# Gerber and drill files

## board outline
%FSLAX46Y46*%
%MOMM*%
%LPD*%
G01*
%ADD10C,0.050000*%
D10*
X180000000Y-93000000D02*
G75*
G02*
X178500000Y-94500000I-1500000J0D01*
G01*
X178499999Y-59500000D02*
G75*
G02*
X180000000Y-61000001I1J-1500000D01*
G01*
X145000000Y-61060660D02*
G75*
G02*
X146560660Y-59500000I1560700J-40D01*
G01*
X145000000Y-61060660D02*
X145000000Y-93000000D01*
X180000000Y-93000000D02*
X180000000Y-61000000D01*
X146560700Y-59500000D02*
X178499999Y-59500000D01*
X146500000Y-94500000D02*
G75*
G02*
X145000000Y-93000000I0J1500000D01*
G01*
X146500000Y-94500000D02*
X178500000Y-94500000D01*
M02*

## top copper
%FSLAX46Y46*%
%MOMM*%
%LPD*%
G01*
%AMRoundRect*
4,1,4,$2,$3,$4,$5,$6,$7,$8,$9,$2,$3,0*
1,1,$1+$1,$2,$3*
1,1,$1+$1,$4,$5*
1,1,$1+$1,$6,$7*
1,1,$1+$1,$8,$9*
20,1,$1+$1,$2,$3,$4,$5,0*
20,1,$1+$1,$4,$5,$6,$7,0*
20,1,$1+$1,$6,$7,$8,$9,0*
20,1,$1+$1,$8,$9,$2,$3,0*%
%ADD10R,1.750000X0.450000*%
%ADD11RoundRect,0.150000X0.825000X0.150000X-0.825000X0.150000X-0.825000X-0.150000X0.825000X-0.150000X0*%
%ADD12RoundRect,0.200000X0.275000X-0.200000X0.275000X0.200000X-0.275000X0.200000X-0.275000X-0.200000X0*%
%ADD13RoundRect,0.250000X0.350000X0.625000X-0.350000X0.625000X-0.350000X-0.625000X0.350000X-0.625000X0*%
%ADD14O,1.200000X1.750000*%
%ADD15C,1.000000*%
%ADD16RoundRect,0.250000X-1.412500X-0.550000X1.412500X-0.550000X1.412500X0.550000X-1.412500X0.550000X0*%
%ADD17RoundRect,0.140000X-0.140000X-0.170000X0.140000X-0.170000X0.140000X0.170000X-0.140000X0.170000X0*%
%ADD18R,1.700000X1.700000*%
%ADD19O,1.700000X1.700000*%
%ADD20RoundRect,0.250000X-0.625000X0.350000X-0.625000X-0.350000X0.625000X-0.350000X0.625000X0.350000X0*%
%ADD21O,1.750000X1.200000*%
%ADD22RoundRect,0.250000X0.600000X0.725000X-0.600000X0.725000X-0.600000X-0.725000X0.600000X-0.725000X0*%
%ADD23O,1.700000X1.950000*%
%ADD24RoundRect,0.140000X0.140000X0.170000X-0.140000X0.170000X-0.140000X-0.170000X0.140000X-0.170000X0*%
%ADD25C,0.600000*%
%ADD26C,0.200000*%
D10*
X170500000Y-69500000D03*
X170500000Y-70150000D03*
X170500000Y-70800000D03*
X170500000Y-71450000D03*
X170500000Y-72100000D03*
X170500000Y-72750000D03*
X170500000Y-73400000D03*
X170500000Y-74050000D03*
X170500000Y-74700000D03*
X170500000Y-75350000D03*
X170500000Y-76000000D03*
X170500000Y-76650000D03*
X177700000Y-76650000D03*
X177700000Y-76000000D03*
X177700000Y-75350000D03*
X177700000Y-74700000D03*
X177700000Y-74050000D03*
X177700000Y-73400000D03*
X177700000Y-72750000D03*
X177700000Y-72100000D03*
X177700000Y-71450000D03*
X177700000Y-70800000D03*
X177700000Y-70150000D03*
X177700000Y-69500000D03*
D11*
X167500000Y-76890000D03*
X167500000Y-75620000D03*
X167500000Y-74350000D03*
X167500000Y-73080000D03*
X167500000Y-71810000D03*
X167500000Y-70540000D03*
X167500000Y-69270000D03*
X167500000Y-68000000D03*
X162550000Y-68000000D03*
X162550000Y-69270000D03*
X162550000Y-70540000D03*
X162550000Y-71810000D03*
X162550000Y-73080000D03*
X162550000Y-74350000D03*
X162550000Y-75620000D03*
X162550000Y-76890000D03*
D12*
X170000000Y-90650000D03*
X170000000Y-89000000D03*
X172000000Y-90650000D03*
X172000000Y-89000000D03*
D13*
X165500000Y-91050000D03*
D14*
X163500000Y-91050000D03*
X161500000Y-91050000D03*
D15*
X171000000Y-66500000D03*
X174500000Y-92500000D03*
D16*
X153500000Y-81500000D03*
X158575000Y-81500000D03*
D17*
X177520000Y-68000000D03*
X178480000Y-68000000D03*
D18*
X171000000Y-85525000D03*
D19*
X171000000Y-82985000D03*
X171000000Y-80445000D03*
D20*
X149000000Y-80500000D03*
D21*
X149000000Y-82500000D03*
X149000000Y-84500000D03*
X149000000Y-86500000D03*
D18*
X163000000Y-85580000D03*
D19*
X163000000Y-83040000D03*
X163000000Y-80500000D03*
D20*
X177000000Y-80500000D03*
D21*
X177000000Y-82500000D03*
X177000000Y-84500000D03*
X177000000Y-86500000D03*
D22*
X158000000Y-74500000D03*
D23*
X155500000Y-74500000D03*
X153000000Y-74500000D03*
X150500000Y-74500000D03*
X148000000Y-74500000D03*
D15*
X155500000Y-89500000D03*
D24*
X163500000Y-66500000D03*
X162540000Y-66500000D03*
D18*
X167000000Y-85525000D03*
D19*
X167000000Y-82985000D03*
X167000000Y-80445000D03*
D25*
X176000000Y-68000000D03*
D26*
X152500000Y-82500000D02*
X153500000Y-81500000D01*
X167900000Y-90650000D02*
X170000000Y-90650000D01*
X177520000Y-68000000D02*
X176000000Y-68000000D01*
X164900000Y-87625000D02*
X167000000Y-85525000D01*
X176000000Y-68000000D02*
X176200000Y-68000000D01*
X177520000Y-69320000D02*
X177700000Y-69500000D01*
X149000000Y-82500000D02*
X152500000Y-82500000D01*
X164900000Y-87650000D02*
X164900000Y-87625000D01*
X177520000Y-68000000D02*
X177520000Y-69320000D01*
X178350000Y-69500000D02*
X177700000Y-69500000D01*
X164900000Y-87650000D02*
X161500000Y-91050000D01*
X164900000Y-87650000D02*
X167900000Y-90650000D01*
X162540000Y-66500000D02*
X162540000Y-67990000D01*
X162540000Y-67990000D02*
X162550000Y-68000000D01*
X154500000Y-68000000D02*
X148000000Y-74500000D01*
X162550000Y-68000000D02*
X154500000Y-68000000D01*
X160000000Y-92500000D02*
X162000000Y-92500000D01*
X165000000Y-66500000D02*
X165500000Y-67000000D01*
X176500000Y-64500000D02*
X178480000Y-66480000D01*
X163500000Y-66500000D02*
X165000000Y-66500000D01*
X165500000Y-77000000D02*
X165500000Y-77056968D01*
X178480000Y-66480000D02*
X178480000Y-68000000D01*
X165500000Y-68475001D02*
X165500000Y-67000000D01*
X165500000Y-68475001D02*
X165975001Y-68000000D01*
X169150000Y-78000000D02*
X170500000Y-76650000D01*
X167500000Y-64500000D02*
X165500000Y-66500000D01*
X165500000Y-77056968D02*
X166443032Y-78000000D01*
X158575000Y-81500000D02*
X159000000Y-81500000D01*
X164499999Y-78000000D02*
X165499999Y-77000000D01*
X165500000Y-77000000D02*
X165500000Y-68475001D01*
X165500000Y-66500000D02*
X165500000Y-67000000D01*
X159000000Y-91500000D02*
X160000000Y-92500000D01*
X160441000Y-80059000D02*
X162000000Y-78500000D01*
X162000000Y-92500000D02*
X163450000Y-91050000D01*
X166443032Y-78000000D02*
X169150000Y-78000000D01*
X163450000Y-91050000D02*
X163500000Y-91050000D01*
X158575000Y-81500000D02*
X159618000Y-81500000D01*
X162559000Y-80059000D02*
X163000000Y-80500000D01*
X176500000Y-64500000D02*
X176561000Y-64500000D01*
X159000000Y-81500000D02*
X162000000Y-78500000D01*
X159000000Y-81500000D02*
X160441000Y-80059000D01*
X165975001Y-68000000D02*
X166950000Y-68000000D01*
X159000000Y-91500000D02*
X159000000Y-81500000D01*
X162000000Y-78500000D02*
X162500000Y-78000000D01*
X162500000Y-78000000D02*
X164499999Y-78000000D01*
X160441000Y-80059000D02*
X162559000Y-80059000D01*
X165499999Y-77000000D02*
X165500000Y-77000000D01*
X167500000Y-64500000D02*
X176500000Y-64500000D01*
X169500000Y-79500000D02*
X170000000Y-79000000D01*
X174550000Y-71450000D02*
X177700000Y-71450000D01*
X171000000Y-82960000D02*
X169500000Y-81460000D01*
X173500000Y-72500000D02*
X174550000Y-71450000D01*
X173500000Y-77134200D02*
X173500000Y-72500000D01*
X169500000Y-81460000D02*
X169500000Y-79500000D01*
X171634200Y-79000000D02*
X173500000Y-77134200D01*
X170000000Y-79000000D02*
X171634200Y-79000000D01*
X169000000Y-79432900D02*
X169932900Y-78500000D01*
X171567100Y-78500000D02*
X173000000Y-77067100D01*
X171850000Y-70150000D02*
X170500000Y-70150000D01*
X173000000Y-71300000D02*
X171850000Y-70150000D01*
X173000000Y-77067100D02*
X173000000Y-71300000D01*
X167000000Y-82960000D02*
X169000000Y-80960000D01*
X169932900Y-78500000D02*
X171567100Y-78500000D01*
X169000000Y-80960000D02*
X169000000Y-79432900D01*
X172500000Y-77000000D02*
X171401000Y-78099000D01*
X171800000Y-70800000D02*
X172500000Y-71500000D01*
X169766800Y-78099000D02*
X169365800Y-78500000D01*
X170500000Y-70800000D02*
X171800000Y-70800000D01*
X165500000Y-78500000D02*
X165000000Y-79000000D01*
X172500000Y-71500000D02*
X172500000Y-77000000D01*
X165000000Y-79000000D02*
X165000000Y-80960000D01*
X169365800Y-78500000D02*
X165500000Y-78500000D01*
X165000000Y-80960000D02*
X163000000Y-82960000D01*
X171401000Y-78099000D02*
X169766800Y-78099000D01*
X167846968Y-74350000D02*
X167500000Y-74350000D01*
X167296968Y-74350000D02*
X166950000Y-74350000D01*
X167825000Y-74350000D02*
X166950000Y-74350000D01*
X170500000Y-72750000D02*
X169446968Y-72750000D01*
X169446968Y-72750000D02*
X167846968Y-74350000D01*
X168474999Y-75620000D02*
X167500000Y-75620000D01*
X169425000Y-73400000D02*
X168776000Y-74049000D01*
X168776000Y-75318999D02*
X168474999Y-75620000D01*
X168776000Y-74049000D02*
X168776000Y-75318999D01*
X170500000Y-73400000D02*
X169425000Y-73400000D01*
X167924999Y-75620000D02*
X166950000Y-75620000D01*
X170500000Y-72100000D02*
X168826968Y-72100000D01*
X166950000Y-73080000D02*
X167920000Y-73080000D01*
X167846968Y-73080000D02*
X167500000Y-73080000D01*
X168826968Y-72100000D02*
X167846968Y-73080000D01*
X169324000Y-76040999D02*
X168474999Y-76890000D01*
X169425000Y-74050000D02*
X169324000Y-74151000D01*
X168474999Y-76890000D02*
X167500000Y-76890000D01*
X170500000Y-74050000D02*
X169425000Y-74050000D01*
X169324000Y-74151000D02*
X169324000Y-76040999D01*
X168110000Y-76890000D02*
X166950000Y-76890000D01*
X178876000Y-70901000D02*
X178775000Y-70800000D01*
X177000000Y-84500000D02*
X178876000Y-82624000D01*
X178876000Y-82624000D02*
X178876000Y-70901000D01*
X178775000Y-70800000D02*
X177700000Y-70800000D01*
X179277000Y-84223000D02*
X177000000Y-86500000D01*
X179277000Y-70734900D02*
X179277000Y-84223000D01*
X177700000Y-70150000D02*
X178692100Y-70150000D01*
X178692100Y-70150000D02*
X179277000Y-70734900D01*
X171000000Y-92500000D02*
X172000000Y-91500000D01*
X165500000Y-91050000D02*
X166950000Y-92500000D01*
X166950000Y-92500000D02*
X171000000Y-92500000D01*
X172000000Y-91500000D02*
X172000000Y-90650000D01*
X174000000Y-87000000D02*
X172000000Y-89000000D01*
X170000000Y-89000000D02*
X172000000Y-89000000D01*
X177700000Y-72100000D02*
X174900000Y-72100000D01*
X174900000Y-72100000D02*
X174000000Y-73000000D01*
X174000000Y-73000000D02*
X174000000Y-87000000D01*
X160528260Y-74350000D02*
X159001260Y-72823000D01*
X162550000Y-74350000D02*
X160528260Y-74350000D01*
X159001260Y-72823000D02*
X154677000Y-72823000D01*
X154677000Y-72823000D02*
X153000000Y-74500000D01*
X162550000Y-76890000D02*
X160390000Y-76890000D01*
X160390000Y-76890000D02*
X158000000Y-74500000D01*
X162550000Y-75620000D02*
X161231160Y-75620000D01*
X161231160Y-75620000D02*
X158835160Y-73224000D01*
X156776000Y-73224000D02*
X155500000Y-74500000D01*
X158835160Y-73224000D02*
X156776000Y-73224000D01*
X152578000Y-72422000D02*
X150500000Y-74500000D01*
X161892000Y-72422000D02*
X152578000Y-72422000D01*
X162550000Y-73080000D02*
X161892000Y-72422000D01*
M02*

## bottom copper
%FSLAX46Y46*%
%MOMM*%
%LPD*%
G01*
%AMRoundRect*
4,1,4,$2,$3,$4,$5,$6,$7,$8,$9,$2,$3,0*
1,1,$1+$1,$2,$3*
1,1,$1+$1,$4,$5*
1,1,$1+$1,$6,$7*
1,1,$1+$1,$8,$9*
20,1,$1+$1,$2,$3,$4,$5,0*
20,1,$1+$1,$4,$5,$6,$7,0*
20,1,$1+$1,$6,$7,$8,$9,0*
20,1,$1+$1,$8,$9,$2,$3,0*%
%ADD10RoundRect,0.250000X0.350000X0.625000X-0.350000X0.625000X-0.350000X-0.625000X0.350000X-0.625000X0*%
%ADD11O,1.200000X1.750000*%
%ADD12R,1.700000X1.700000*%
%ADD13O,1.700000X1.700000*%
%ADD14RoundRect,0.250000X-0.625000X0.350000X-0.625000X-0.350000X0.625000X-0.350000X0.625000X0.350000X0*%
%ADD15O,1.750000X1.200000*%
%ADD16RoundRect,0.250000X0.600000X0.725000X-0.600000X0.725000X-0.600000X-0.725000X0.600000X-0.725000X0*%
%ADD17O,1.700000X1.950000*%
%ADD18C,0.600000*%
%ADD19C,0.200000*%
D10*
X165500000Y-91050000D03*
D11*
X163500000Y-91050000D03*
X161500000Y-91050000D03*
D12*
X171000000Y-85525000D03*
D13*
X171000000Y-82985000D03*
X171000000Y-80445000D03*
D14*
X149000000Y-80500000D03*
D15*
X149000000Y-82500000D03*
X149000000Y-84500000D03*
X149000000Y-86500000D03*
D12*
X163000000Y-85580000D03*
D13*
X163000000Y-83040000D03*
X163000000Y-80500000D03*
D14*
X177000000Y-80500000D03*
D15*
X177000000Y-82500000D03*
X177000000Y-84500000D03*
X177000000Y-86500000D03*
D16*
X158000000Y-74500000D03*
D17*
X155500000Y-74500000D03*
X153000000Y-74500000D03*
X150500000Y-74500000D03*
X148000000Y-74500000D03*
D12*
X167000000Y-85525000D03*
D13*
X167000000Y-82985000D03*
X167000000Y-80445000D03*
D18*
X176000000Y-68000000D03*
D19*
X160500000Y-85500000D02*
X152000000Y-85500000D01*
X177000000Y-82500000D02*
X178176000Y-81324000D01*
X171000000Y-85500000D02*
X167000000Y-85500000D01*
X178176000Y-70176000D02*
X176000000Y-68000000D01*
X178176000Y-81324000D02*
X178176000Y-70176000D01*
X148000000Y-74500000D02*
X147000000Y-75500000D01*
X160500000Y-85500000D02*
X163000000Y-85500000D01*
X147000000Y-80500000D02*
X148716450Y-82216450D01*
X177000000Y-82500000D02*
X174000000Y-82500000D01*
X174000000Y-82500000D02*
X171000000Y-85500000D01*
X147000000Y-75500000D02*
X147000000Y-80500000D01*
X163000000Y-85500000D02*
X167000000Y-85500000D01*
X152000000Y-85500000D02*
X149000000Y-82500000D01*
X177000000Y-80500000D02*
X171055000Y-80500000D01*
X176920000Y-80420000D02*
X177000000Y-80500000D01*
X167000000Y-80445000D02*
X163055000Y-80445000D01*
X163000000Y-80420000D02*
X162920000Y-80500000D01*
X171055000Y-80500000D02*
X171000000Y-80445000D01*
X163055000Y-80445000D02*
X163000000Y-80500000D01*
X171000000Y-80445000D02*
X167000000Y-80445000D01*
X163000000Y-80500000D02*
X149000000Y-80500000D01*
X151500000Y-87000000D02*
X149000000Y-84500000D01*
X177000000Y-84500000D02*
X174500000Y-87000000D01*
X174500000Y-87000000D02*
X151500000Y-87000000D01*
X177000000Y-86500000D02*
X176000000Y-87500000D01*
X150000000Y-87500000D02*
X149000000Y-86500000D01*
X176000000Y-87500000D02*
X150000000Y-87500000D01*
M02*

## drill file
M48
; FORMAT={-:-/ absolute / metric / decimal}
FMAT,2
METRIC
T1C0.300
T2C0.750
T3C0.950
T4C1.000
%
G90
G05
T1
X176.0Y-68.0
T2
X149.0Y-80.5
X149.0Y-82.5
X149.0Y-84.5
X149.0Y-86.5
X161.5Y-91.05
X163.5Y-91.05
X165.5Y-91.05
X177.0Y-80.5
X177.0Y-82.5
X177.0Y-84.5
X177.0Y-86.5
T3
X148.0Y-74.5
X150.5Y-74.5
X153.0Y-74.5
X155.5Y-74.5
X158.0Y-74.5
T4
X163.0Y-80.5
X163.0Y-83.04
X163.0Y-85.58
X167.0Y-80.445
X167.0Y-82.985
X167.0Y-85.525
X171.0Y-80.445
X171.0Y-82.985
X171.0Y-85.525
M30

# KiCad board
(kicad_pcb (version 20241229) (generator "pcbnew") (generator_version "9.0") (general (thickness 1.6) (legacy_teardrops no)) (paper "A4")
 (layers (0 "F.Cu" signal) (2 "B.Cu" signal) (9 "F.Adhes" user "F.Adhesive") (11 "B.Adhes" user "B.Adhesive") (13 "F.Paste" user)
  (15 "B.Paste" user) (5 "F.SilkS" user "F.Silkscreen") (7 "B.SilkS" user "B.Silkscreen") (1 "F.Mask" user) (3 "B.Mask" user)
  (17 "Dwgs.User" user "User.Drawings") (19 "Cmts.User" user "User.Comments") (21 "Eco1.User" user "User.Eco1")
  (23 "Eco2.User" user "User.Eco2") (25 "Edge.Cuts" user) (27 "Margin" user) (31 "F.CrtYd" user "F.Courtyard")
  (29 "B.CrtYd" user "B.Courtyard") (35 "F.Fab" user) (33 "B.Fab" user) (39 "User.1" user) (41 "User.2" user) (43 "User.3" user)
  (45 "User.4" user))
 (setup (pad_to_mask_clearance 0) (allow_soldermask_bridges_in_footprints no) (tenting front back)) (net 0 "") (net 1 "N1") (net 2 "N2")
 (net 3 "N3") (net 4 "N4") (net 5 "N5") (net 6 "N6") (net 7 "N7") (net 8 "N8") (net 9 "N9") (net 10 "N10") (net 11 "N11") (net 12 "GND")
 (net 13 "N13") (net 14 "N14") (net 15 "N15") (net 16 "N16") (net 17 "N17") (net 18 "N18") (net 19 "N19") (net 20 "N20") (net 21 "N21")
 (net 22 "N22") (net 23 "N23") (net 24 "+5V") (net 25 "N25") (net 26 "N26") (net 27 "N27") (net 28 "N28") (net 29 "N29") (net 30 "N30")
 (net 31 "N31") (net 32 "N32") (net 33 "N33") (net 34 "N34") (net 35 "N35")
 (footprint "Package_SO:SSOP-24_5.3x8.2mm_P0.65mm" (layer "F.Cu") (at 174.1 73.075)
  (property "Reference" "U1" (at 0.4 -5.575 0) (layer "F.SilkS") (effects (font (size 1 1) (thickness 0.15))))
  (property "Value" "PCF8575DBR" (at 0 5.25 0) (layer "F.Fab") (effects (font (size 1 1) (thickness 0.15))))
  (pad "1" smd rect (at -3.6 -3.575) (size 1.75 0.45) (layers "F.Cu" "F.Mask" "F.Paste") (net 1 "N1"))
  (pad "2" smd rect (at -3.6 -2.925) (size 1.75 0.45) (layers "F.Cu" "F.Mask" "F.Paste") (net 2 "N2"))
  (pad "3" smd rect (at -3.6 -2.275) (size 1.75 0.45) (layers "F.Cu" "F.Mask" "F.Paste") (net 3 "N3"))
  (pad "4" smd rect (at -3.6 -1.625) (size 1.75 0.45) (layers "F.Cu" "F.Mask" "F.Paste") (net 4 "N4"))
  (pad "5" smd rect (at -3.6 -0.975) (size 1.75 0.45) (layers "F.Cu" "F.Mask" "F.Paste") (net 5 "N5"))
  (pad "6" smd rect (at -3.6 -0.325) (size 1.75 0.45) (layers "F.Cu" "F.Mask" "F.Paste") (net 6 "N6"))
  (pad "7" smd rect (at -3.6 0.325) (size 1.75 0.45) (layers "F.Cu" "F.Mask" "F.Paste") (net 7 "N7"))
  (pad "8" smd rect (at -3.6 0.975) (size 1.75 0.45) (layers "F.Cu" "F.Mask" "F.Paste") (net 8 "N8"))
  (pad "9" smd rect (at -3.6 1.625) (size 1.75 0.45) (layers "F.Cu" "F.Mask" "F.Paste") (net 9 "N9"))
  (pad "10" smd rect (at -3.6 2.275) (size 1.75 0.45) (layers "F.Cu" "F.Mask" "F.Paste") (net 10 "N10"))
  (pad "11" smd rect (at -3.6 2.925) (size 1.75 0.45) (layers "F.Cu" "F.Mask" "F.Paste") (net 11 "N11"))
  (pad "12" smd rect (at -3.6 3.575) (size 1.75 0.45) (layers "F.Cu" "F.Mask" "F.Paste") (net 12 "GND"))
  (pad "13" smd rect (at 3.6 3.575) (size 1.75 0.45) (layers "F.Cu" "F.Mask" "F.Paste") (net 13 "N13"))
  (pad "14" smd rect (at 3.6 2.925) (size 1.75 0.45) (layers "F.Cu" "F.Mask" "F.Paste") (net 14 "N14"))
  (pad "15" smd rect (at 3.6 2.275) (size 1.75 0.45) (layers "F.Cu" "F.Mask" "F.Paste") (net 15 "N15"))
  (pad "16" smd rect (at 3.6 1.625) (size 1.75 0.45) (layers "F.Cu" "F.Mask" "F.Paste") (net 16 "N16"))
  (pad "17" smd rect (at 3.6 0.975) (size 1.75 0.45) (layers "F.Cu" "F.Mask" "F.Paste") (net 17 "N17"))
  (pad "18" smd rect (at 3.6 0.325) (size 1.75 0.45) (layers "F.Cu" "F.Mask" "F.Paste") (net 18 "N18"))
  (pad "19" smd rect (at 3.6 -0.325) (size 1.75 0.45) (layers "F.Cu" "F.Mask" "F.Paste") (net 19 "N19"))
  (pad "20" smd rect (at 3.6 -0.975) (size 1.75 0.45) (layers "F.Cu" "F.Mask" "F.Paste") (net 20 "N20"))
  (pad "21" smd rect (at 3.6 -1.625) (size 1.75 0.45) (layers "F.Cu" "F.Mask" "F.Paste") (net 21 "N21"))
  (pad "22" smd rect (at 3.6 -2.275) (size 1.75 0.45) (layers "F.Cu" "F.Mask" "F.Paste") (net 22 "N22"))
  (pad "23" smd rect (at 3.6 -2.925) (size 1.75 0.45) (layers "F.Cu" "F.Mask" "F.Paste") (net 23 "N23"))
  (pad "24" smd rect (at 3.6 -3.575) (size 1.75 0.45) (layers "F.Cu" "F.Mask" "F.Paste") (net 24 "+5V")))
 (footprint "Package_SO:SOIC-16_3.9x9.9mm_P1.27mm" (layer "F.Cu") (at 165.025 72.445 180)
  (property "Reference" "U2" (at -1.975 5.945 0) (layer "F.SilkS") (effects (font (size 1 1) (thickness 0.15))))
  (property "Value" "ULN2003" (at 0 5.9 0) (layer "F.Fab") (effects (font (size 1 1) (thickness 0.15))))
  (pad "1" smd roundrect (at -2.475 -4.445 180) (size 1.95 0.6) (layers "F.Cu" "F.Mask" "F.Paste") (roundrect_rratio 0.25) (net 8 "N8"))
  (pad "2" smd roundrect (at -2.475 -3.175 180) (size 1.95 0.6) (layers "F.Cu" "F.Mask" "F.Paste") (roundrect_rratio 0.25) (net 7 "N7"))
  (pad "3" smd roundrect (at -2.475 -1.905 180) (size 1.95 0.6) (layers "F.Cu" "F.Mask" "F.Paste") (roundrect_rratio 0.25) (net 6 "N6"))
  (pad "4" smd roundrect (at -2.475 -0.635 180) (size 1.95 0.6) (layers "F.Cu" "F.Mask" "F.Paste") (roundrect_rratio 0.25) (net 5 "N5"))
  (pad "5" smd roundrect (at -2.475 0.635 180) (size 1.95 0.6) (layers "F.Cu" "F.Mask" "F.Paste") (roundrect_rratio 0.25) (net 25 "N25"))
  (pad "6" smd roundrect (at -2.475 1.905 180) (size 1.95 0.6) (layers "F.Cu" "F.Mask" "F.Paste") (roundrect_rratio 0.25) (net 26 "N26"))
  (pad "7" smd roundrect (at -2.475 3.175 180) (size 1.95 0.6) (layers "F.Cu" "F.Mask" "F.Paste") (roundrect_rratio 0.25) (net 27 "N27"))
  (pad "8" smd roundrect (at -2.475 4.445 180) (size 1.95 0.6) (layers "F.Cu" "F.Mask" "F.Paste") (roundrect_rratio 0.25) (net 12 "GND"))
  (pad "9" smd roundrect (at 2.475 4.445 180) (size 1.95 0.6) (layers "F.Cu" "F.Mask" "F.Paste") (roundrect_rratio 0.25) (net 24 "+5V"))
  (pad "10" smd roundrect (at 2.475 3.175 180) (size 1.95 0.6) (layers "F.Cu" "F.Mask" "F.Paste") (roundrect_rratio 0.25) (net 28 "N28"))
  (pad "11" smd roundrect (at 2.475 1.905 180) (size 1.95 0.6) (layers "F.Cu" "F.Mask" "F.Paste") (roundrect_rratio 0.25) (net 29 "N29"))
  (pad "12" smd roundrect (at 2.475 0.635 180) (size 1.95 0.6) (layers "F.Cu" "F.Mask" "F.Paste") (roundrect_rratio 0.25) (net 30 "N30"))
  (pad "13" smd roundrect (at 2.475 -0.635 180) (size 1.95 0.6) (layers "F.Cu" "F.Mask" "F.Paste") (roundrect_rratio 0.25) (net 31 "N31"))
  (pad "14" smd roundrect (at 2.475 -1.905 180) (size 1.95 0.6) (layers "F.Cu" "F.Mask" "F.Paste") (roundrect_rratio 0.25) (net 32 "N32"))
  (pad "15" smd roundrect (at 2.475 -3.175 180) (size 1.95 0.6) (layers "F.Cu" "F.Mask" "F.Paste") (roundrect_rratio 0.25) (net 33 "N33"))
  (pad "16" smd roundrect (at 2.475 -4.445 180) (size 1.95 0.6) (layers "F.Cu" "F.Mask" "F.Paste") (roundrect_rratio 0.25) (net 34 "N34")))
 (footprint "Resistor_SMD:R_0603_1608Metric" (layer "F.Cu") (at 170 89.825 90)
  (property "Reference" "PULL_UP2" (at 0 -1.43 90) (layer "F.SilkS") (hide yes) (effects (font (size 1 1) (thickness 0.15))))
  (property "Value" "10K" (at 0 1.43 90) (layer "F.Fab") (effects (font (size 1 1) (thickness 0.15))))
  (pad "1" smd roundrect (at -0.825 0 90) (size 0.8 0.95) (layers "F.Cu" "F.Mask" "F.Paste") (roundrect_rratio 0.25) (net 24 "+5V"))
  (pad "2" smd roundrect (at 0.825 0 90) (size 0.8 0.95) (layers "F.Cu" "F.Mask" "F.Paste") (roundrect_rratio 0.25) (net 20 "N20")))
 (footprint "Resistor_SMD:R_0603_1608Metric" (layer "F.Cu") (at 172 89.825 90)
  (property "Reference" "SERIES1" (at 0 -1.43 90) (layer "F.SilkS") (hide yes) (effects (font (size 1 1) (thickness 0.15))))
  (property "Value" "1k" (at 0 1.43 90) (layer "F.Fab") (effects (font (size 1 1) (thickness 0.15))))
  (pad "1" smd roundrect (at -0.825 0 90) (size 0.8 0.95) (layers "F.Cu" "F.Mask" "F.Paste") (roundrect_rratio 0.25) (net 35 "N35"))
  (pad "2" smd roundrect (at 0.825 0 90) (size 0.8 0.95) (layers "F.Cu" "F.Mask" "F.Paste") (roundrect_rratio 0.25) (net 20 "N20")))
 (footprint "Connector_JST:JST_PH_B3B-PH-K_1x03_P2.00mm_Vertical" (layer "F.Cu") (at 165.5 91.05 180)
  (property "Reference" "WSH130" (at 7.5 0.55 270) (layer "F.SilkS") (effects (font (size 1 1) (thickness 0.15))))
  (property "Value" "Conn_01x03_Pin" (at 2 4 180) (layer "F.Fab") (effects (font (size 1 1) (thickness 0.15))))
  (pad "1" thru_hole roundrect (at 0 0 180) (size 1.2 1.75) (drill 0.75) (layers "*.Cu" "*.Mask") (remove_unused_layers no)
   (roundrect_rratio 0.208333) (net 35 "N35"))
  (pad "2" thru_hole oval (at 2 0 180) (size 1.2 1.75) (drill 0.75) (layers "*.Cu" "*.Mask") (remove_unused_layers no) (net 12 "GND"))
  (pad "3" thru_hole oval (at 4 0 180) (size 1.2 1.75) (drill 0.75) (layers "*.Cu" "*.Mask") (remove_unused_layers no) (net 24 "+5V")))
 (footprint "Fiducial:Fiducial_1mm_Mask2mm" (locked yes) (layer "F.Cu") (at 171 66.5)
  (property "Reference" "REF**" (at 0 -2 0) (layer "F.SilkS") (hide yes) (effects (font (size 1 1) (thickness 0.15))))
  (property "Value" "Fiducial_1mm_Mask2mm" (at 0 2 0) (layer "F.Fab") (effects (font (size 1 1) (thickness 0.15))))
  (pad "" smd circle (at 0 0) (size 1 1) (layers "F.Cu" "F.Mask") (solder_mask_margin 0.5) (clearance 0.5)))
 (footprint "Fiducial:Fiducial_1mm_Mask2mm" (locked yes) (layer "F.Cu") (at 174.5 92.5)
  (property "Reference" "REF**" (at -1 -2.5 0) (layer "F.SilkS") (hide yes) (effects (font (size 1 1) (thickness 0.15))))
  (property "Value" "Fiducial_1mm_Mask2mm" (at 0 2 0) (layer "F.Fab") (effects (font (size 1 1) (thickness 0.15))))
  (pad "" smd circle (at 0 0) (size 1 1) (layers "F.Cu" "F.Mask") (solder_mask_margin 0.5) (clearance 0.5)))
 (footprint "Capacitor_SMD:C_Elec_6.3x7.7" (layer "F.Cu") (at 156.0375 81.5)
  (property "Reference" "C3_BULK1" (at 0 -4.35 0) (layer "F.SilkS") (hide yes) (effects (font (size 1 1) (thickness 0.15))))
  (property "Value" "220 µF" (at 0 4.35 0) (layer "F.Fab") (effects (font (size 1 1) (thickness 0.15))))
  (pad "1" smd roundrect (at -2.5375 0) (size 3.325 1.6) (layers "F.Cu" "F.Mask" "F.Paste") (roundrect_rratio 0.15625) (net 24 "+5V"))
  (pad "2" smd roundrect (at 2.5375 0) (size 3.325 1.6) (layers "F.Cu" "F.Mask" "F.Paste") (roundrect_rratio 0.15625) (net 12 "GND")))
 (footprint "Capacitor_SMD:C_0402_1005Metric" (layer "F.Cu") (at 178 68)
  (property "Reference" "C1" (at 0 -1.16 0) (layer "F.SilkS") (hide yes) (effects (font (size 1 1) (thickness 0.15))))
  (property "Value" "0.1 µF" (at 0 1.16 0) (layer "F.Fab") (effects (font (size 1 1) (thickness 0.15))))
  (pad "1" smd roundrect (at -0.48 0) (size 0.56 0.62) (layers "F.Cu" "F.Mask" "F.Paste") (roundrect_rratio 0.25) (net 24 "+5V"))
  (pad "2" smd roundrect (at 0.48 0) (size 0.56 0.62) (layers "F.Cu" "F.Mask" "F.Paste") (roundrect_rratio 0.25) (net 12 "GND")))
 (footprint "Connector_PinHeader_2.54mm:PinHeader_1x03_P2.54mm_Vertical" (layer "F.Cu") (at 171 85.525 180)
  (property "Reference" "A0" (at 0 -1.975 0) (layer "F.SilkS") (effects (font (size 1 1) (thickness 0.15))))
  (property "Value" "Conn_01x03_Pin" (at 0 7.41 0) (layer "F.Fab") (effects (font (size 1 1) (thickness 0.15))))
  (pad "1" thru_hole rect (at 0 0 180) (size 1.7 1.7) (drill 1) (layers "*.Cu" "*.Mask") (remove_unused_layers no) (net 24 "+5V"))
  (pad "2" thru_hole oval (at 0 2.54 180) (size 1.7 1.7) (drill 1) (layers "*.Cu" "*.Mask") (remove_unused_layers no) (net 21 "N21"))
  (pad "3" thru_hole oval (at 0 5.08 180) (size 1.7 1.7) (drill 1) (layers "*.Cu" "*.Mask") (remove_unused_layers no) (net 12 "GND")))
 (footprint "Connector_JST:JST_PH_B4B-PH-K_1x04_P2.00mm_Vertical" (layer "F.Cu") (at 149 80.5 -90)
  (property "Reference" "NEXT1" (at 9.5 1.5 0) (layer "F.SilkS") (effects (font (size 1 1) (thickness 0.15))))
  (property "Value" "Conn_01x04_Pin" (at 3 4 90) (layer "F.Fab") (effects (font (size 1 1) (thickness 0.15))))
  (pad "1" thru_hole roundrect (at 0 0 270) (size 1.2 1.75) (drill 0.75) (layers "*.Cu" "*.Mask") (remove_unused_layers no)
   (roundrect_rratio 0.208333) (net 12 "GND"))
  (pad "2" thru_hole oval (at 2 0 270) (size 1.2 1.75) (drill 0.75) (layers "*.Cu" "*.Mask") (remove_unused_layers no) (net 24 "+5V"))
  (pad "3" thru_hole oval (at 4 0 270) (size 1.2 1.75) (drill 0.75) (layers "*.Cu" "*.Mask") (remove_unused_layers no) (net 22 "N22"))
  (pad "4" thru_hole oval (at 6 0 270) (size 1.2 1.75) (drill 0.75) (layers "*.Cu" "*.Mask") (remove_unused_layers no) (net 23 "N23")))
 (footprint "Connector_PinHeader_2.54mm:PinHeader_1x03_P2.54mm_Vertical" (layer "F.Cu") (at 163 85.58 180)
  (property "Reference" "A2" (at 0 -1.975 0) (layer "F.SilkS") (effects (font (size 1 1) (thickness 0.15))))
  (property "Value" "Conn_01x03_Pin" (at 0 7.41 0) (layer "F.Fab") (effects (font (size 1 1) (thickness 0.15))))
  (pad "1" thru_hole rect (at 0 0 180) (size 1.7 1.7) (drill 1) (layers "*.Cu" "*.Mask") (remove_unused_layers no) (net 24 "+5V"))
  (pad "2" thru_hole oval (at 0 2.54 180) (size 1.7 1.7) (drill 1) (layers "*.Cu" "*.Mask") (remove_unused_layers no) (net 3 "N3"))
  (pad "3" thru_hole oval (at 0 5.08 180) (size 1.7 1.7) (drill 1) (layers "*.Cu" "*.Mask") (remove_unused_layers no) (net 12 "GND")))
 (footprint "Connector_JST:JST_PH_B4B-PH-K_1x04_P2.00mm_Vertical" (layer "F.Cu") (at 177 80.5 -90)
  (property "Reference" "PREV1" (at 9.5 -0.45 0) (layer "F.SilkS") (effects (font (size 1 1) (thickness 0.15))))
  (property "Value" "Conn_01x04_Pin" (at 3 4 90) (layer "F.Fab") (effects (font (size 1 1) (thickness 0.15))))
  (pad "1" thru_hole roundrect (at 0 0 270) (size 1.2 1.75) (drill 0.75) (layers "*.Cu" "*.Mask") (remove_unused_layers no)
   (roundrect_rratio 0.208333) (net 12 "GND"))
  (pad "2" thru_hole oval (at 2 0 270) (size 1.2 1.75) (drill 0.75) (layers "*.Cu" "*.Mask") (remove_unused_layers no) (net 24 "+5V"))
  (pad "3" thru_hole oval (at 4 0 270) (size 1.2 1.75) (drill 0.75) (layers "*.Cu" "*.Mask") (remove_unused_layers no) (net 22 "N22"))
  (pad "4" thru_hole oval (at 6 0 270) (size 1.2 1.75) (drill 0.75) (layers "*.Cu" "*.Mask") (remove_unused_layers no) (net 23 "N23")))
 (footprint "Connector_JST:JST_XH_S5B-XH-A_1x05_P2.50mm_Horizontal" (layer "F.Cu") (at 158 74.5 180)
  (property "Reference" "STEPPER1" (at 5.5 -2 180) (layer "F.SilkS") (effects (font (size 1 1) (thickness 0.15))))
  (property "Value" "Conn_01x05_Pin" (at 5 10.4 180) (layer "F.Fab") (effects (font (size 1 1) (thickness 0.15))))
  (pad "1" thru_hole roundrect (at 0 0 180) (size 1.7 1.95) (drill 0.95) (layers "*.Cu" "*.Mask") (remove_unused_layers no)
   (roundrect_rratio 0.147059) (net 34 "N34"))
  (pad "2" thru_hole oval (at 2.5 0 180) (size 1.7 1.95) (drill 0.95) (layers "*.Cu" "*.Mask") (remove_unused_layers no) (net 33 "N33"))
  (pad "3" thru_hole oval (at 5 0 180) (size 1.7 1.95) (drill 0.95) (layers "*.Cu" "*.Mask") (remove_unused_layers no) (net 32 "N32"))
  (pad "4" thru_hole oval (at 7.5 0 180) (size 1.7 1.95) (drill 0.95) (layers "*.Cu" "*.Mask") (remove_unused_layers no) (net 31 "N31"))
  (pad "5" thru_hole oval (at 10 0 180) (size 1.7 1.95) (drill 0.95) (layers "*.Cu" "*.Mask") (remove_unused_layers no) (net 24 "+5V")))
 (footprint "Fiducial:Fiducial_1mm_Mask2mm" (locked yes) (layer "F.Cu") (at 155.5 89.5)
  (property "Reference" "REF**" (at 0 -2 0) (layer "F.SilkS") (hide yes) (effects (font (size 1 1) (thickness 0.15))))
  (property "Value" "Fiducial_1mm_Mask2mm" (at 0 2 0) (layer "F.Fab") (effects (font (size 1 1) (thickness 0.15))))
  (pad "" smd circle (at 0 0) (size 1 1) (layers "F.Cu" "F.Mask") (solder_mask_margin 0.5) (clearance 0.5)))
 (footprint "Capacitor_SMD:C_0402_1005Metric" (layer "F.Cu") (at 163.02 66.5 180)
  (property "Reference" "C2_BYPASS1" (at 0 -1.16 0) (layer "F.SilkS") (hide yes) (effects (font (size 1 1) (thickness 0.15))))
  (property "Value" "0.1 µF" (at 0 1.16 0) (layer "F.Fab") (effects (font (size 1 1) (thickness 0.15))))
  (pad "1" smd roundrect (at -0.48 0 180) (size 0.56 0.62) (layers "F.Cu" "F.Mask" "F.Paste") (roundrect_rratio 0.25) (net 12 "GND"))
  (pad "2" smd roundrect (at 0.48 0 180) (size 0.56 0.62) (layers "F.Cu" "F.Mask" "F.Paste") (roundrect_rratio 0.25) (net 24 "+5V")))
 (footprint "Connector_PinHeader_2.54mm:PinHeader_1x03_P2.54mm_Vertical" (layer "F.Cu") (at 167 85.525 180)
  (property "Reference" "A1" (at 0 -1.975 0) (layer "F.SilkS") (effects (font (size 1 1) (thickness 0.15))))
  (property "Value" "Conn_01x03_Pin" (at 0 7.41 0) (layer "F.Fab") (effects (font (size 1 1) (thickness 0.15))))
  (pad "1" thru_hole rect (at 0 0 180) (size 1.7 1.7) (drill 1) (layers "*.Cu" "*.Mask") (remove_unused_layers no) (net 24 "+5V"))
  (pad "2" thru_hole oval (at 0 2.54 180) (size 1.7 1.7) (drill 1) (layers "*.Cu" "*.Mask") (remove_unused_layers no) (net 2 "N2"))
  (pad "3" thru_hole oval (at 0 5.08 180) (size 1.7 1.7) (drill 1) (layers "*.Cu" "*.Mask") (remove_unused_layers no) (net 12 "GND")))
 (gr_arc (start 180 93) (mid 179.56066 94.06066) (end 178.5 94.5) (stroke (width 0.05) (type default)) (layer "Edge.Cuts"))
 (gr_arc (start 178.499999 59.5) (mid 179.56066 59.93934) (end 180 61.000001) (stroke (width 0.05) (type default)) (layer "Edge.Cuts"))
 (gr_arc (start 145 61.06066) (mid 145.457107 59.957107) (end 146.56066 59.5) (stroke (width 0.05) (type default)) (layer "Edge.Cuts"))
 (gr_line (start 145 61.06066) (end 145 93) (stroke (width 0.05) (type default)) (layer "Edge.Cuts"))
 (gr_line (start 180 93) (end 180 61) (stroke (width 0.05) (type default)) (layer "Edge.Cuts"))
 (gr_line (start 146.5607 59.5) (end 178.499999 59.5) (stroke (width 0.05) (type default)) (layer "Edge.Cuts"))
 (gr_arc (start 146.5 94.5) (mid 145.43934 94.06066) (end 145 93) (stroke (width 0.05) (type default)) (layer "Edge.Cuts"))
 (gr_line (start 146.5 94.5) (end 178.5 94.5) (stroke (width 0.05) (type default)) (layer "Edge.Cuts"))
 (segment (start 152.5 82.5) (end 153.5 81.5) (width 0.2) (layer "F.Cu") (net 24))
 (segment (start 167.9 90.65) (end 170 90.65) (width 0.2) (layer "F.Cu") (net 24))
 (segment (start 177.52 68) (end 176 68) (width 0.2) (layer "F.Cu") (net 24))
 (segment (start 164.9 87.625) (end 167 85.525) (width 0.2) (layer "F.Cu") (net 24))
 (segment (start 176 68) (end 176.2 68) (width 0.2) (layer "F.Cu") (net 24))
 (segment (start 177.52 69.32) (end 177.7 69.5) (width 0.2) (layer "F.Cu") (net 24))
 (segment (start 149 82.5) (end 152.5 82.5) (width 0.2) (layer "F.Cu") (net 24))
 (segment (start 164.9 87.65) (end 164.9 87.625) (width 0.2) (layer "F.Cu") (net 24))
 (segment (start 177.52 68) (end 177.52 69.32) (width 0.2) (layer "F.Cu") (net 24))
 (segment (start 178.35 69.5) (end 177.7 69.5) (width 0.2) (layer "F.Cu") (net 24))
 (segment (start 164.9 87.65) (end 161.5 91.05) (width 0.2) (layer "F.Cu") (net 24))
 (segment (start 164.9 87.65) (end 167.9 90.65) (width 0.2) (layer "F.Cu") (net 24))
 (segment (start 162.54 66.5) (end 162.54 67.99) (width 0.2) (layer "F.Cu") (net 24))
 (segment (start 162.54 67.99) (end 162.55 68) (width 0.2) (layer "F.Cu") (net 24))
 (segment (start 154.5 68) (end 148 74.5) (width 0.2) (layer "F.Cu") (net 24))
 (segment (start 162.55 68) (end 154.5 68) (width 0.2) (layer "F.Cu") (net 24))
 (via (at 176 68) (size 0.6) (drill 0.3) (layers "F.Cu" "B.Cu") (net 24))
 (segment (start 160.5 85.5) (end 152 85.5) (width 0.2) (layer "B.Cu") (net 24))
 (segment (start 177 82.5) (end 178.176 81.324) (width 0.2) (layer "B.Cu") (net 24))
 (segment (start 171 85.5) (end 167 85.5) (width 0.2) (layer "B.Cu") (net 24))
 (segment (start 178.176 70.176) (end 176 68) (width 0.2) (layer "B.Cu") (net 24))
 (segment (start 178.176 81.324) (end 178.176 70.176) (width 0.2) (layer "B.Cu") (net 24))
 (segment (start 148 74.5) (end 147 75.5) (width 0.2) (layer "B.Cu") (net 24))
 (segment (start 160.5 85.5) (end 163 85.5) (width 0.2) (layer "B.Cu") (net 24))
 (segment (start 147 80.5) (end 148.71645 82.21645) (width 0.2) (layer "B.Cu") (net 24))
 (segment (start 177 82.5) (end 174 82.5) (width 0.2) (layer "B.Cu") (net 24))
 (segment (start 174 82.5) (end 171 85.5) (width 0.2) (layer "B.Cu") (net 24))
 (segment (start 147 75.5) (end 147 80.5) (width 0.2) (layer "B.Cu") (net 24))
 (segment (start 163 85.5) (end 167 85.5) (width 0.2) (layer "B.Cu") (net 24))
 (segment (start 152 85.5) (end 149 82.5) (width 0.2) (layer "B.Cu") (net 24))
 (segment (start 160 92.5) (end 162 92.5) (width 0.2) (layer "F.Cu") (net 12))
 (segment (start 165 66.5) (end 165.5 67) (width 0.2) (layer "F.Cu") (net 12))
 (segment (start 176.5 64.5) (end 178.48 66.48) (width 0.2) (layer "F.Cu") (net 12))
 (segment (start 163.5 66.5) (end 165 66.5) (width 0.2) (layer "F.Cu") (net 12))
 (segment (start 165.5 77) (end 165.5 77.056968) (width 0.2) (layer "F.Cu") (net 12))
 (segment (start 178.48 66.48) (end 178.48 68) (width 0.2) (layer "F.Cu") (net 12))
 (segment (start 165.5 68.475001) (end 165.5 67) (width 0.2) (layer "F.Cu") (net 12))
 (segment (start 165.5 68.475001) (end 165.975001 68) (width 0.2) (layer "F.Cu") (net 12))
 (segment (start 169.15 78) (end 170.5 76.65) (width 0.2) (layer "F.Cu") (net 12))
 (segment (start 167.5 64.5) (end 165.5 66.5) (width 0.2) (layer "F.Cu") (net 12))
 (segment (start 165.5 77.056968) (end 166.443032 78) (width 0.2) (layer "F.Cu") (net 12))
 (segment (start 158.575 81.5) (end 159 81.5) (width 0.2) (layer "F.Cu") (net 12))
 (segment (start 164.499999 78) (end 165.499999 77) (width 0.2) (layer "F.Cu") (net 12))
 (segment (start 165.5 77) (end 165.5 68.475001) (width 0.2) (layer "F.Cu") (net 12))
 (segment (start 165.5 66.5) (end 165.5 67) (width 0.2) (layer "F.Cu") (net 12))
 (segment (start 159 91.5) (end 160 92.5) (width 0.2) (layer "F.Cu") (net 12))
 (segment (start 160.441 80.059) (end 162 78.5) (width 0.2) (layer "F.Cu") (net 12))
 (segment (start 162 92.5) (end 163.45 91.05) (width 0.2) (layer "F.Cu") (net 12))
 (segment (start 166.443032 78) (end 169.15 78) (width 0.2) (layer "F.Cu") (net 12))
 (segment (start 163.45 91.05) (end 163.5 91.05) (width 0.2) (layer "F.Cu") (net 12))
 (segment (start 158.575 81.5) (end 159.618 81.5) (width 0.2) (layer "F.Cu") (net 12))
 (segment (start 162.559 80.059) (end 163 80.5) (width 0.2) (layer "F.Cu") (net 12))
 (segment (start 176.5 64.5) (end 176.561 64.5) (width 0.2) (layer "F.Cu") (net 12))
 (segment (start 159 81.5) (end 162 78.5) (width 0.2) (layer "F.Cu") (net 12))
 (segment (start 159 81.5) (end 160.441 80.059) (width 0.2) (layer "F.Cu") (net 12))
 (segment (start 165.975001 68) (end 166.95 68) (width 0.2) (layer "F.Cu") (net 12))
 (segment (start 159 91.5) (end 159 81.5) (width 0.2) (layer "F.Cu") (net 12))
 (segment (start 162 78.5) (end 162.5 78) (width 0.2) (layer "F.Cu") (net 12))
 (segment (start 162.5 78) (end 164.499999 78) (width 0.2) (layer "F.Cu") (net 12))
 (segment (start 160.441 80.059) (end 162.559 80.059) (width 0.2) (layer "F.Cu") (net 12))
 (segment (start 165.499999 77) (end 165.5 77) (width 0.2) (layer "F.Cu") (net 12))
 (segment (start 167.5 64.5) (end 176.5 64.5) (width 0.2) (layer "F.Cu") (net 12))
 (segment (start 177 80.5) (end 171.055 80.5) (width 0.2) (layer "B.Cu") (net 12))
 (segment (start 176.92 80.42) (end 177 80.5) (width 0.2) (layer "B.Cu") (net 12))
 (segment (start 167 80.445) (end 163.055 80.445) (width 0.2) (layer "B.Cu") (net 12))
 (segment (start 163 80.42) (end 162.92 80.5) (width 0.2) (layer "B.Cu") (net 12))
 (segment (start 171.055 80.5) (end 171 80.445) (width 0.2) (layer "B.Cu") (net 12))
 (segment (start 163.055 80.445) (end 163 80.5) (width 0.2) (layer "B.Cu") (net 12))
 (segment (start 171 80.445) (end 167 80.445) (width 0.2) (layer "B.Cu") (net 12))
 (segment (start 163 80.5) (end 149 80.5) (width 0.2) (layer "B.Cu") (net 12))
 (segment (start 169.5 79.5) (end 170 79) (width 0.2) (layer "F.Cu") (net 21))
 (segment (start 174.55 71.45) (end 177.7 71.45) (width 0.2) (layer "F.Cu") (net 21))
 (segment (start 171 82.96) (end 169.5 81.46) (width 0.2) (layer "F.Cu") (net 21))
 (segment (start 173.5 72.5) (end 174.55 71.45) (width 0.2) (layer "F.Cu") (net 21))
 (segment (start 173.5 77.1342) (end 173.5 72.5) (width 0.2) (layer "F.Cu") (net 21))
 (segment (start 169.5 81.46) (end 169.5 79.5) (width 0.2) (layer "F.Cu") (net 21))
 (segment (start 171.6342 79) (end 173.5 77.1342) (width 0.2) (layer "F.Cu") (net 21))
 (segment (start 170 79) (end 171.6342 79) (width 0.2) (layer "F.Cu") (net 21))
 (segment (start 169 79.4329) (end 169.9329 78.5) (width 0.2) (layer "F.Cu") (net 2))
 (segment (start 171.5671 78.5) (end 173 77.0671) (width 0.2) (layer "F.Cu") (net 2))
 (segment (start 171.85 70.15) (end 170.5 70.15) (width 0.2) (layer "F.Cu") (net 2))
 (segment (start 173 71.3) (end 171.85 70.15) (width 0.2) (layer "F.Cu") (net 2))
 (segment (start 173 77.0671) (end 173 71.3) (width 0.2) (layer "F.Cu") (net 2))
 (segment (start 167 82.96) (end 169 80.96) (width 0.2) (layer "F.Cu") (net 2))
 (segment (start 169.9329 78.5) (end 171.5671 78.5) (width 0.2) (layer "F.Cu") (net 2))
 (segment (start 169 80.96) (end 169 79.4329) (width 0.2) (layer "F.Cu") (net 2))
 (segment (start 172.5 77) (end 171.401 78.099) (width 0.2) (layer "F.Cu") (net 3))
 (segment (start 171.8 70.8) (end 172.5 71.5) (width 0.2) (layer "F.Cu") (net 3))
 (segment (start 169.7668 78.099) (end 169.3658 78.5) (width 0.2) (layer "F.Cu") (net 3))
 (segment (start 170.5 70.8) (end 171.8 70.8) (width 0.2) (layer "F.Cu") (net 3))
 (segment (start 165.5 78.5) (end 165 79) (width 0.2) (layer "F.Cu") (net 3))
 (segment (start 172.5 71.5) (end 172.5 77) (width 0.2) (layer "F.Cu") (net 3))
 (segment (start 165 79) (end 165 80.96) (width 0.2) (layer "F.Cu") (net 3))
 (segment (start 169.3658 78.5) (end 165.5 78.5) (width 0.2) (layer "F.Cu") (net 3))
 (segment (start 165 80.96) (end 163 82.96) (width 0.2) (layer "F.Cu") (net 3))
 (segment (start 171.401 78.099) (end 169.7668 78.099) (width 0.2) (layer "F.Cu") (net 3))
 (segment (start 167.846968 74.35) (end 167.5 74.35) (width 0.2) (layer "F.Cu") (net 6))
 (segment (start 167.296968 74.35) (end 166.95 74.35) (width 0.2) (layer "F.Cu") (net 6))
 (segment (start 167.825 74.35) (end 166.95 74.35) (width 0.2) (layer "F.Cu") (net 6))
 (segment (start 170.5 72.75) (end 169.446968 72.75) (width 0.2) (layer "F.Cu") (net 6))
 (segment (start 169.446968 72.75) (end 167.846968 74.35) (width 0.2) (layer "F.Cu") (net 6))
 (segment (start 168.474999 75.62) (end 167.5 75.62) (width 0.2) (layer "F.Cu") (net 7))
 (segment (start 169.425 73.4) (end 168.776 74.049) (width 0.2) (layer "F.Cu") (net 7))
 (segment (start 168.776 75.318999) (end 168.474999 75.62) (width 0.2) (layer "F.Cu") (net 7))
 (segment (start 168.776 74.049) (end 168.776 75.318999) (width 0.2) (layer "F.Cu") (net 7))
 (segment (start 170.5 73.4) (end 169.425 73.4) (width 0.2) (layer "F.Cu") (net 7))
 (segment (start 167.924999 75.62) (end 166.95 75.62) (width 0.2) (layer "F.Cu") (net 7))
 (segment (start 170.5 72.1) (end 168.826968 72.1) (width 0.2) (layer "F.Cu") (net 5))
 (segment (start 166.95 73.08) (end 167.92 73.08) (width 0.2) (layer "F.Cu") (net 5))
 (segment (start 167.846968 73.08) (end 167.5 73.08) (width 0.2) (layer "F.Cu") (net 5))
 (segment (start 168.826968 72.1) (end 167.846968 73.08) (width 0.2) (layer "F.Cu") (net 5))
 (segment (start 169.324 76.040999) (end 168.474999 76.89) (width 0.2) (layer "F.Cu") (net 8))
 (segment (start 169.425 74.05) (end 169.324 74.151) (width 0.2) (layer "F.Cu") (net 8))
 (segment (start 168.474999 76.89) (end 167.5 76.89) (width 0.2) (layer "F.Cu") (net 8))
 (segment (start 170.5 74.05) (end 169.425 74.05) (width 0.2) (layer "F.Cu") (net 8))
 (segment (start 169.324 74.151) (end 169.324 76.040999) (width 0.2) (layer "F.Cu") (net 8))
 (segment (start 168.11 76.89) (end 166.95 76.89) (width 0.2) (layer "F.Cu") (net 8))
 (segment (start 178.876 70.901) (end 178.775 70.8) (width 0.2) (layer "F.Cu") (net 22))
 (segment (start 177 84.5) (end 178.876 82.624) (width 0.2) (layer "F.Cu") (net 22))
 (segment (start 178.876 82.624) (end 178.876 70.901) (width 0.2) (layer "F.Cu") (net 22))
 (segment (start 178.775 70.8) (end 177.7 70.8) (width 0.2) (layer "F.Cu") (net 22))
 (segment (start 151.5 87) (end 149 84.5) (width 0.2) (layer "B.Cu") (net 22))
 (segment (start 177 84.5) (end 174.5 87) (width 0.2) (layer "B.Cu") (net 22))
 (segment (start 174.5 87) (end 151.5 87) (width 0.2) (layer "B.Cu") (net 22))
 (segment (start 179.277 84.223) (end 177 86.5) (width 0.2) (layer "F.Cu") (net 23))
 (segment (start 179.277 70.7349) (end 179.277 84.223) (width 0.2) (layer "F.Cu") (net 23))
 (segment (start 177.7 70.15) (end 178.6921 70.15) (width 0.2) (layer "F.Cu") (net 23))
 (segment (start 178.6921 70.15) (end 179.277 70.7349) (width 0.2) (layer "F.Cu") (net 23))
 (segment (start 177 86.5) (end 176 87.5) (width 0.2) (layer "B.Cu") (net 23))
 (segment (start 150 87.5) (end 149 86.5) (width 0.2) (layer "B.Cu") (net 23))
 (segment (start 176 87.5) (end 150 87.5) (width 0.2) (layer "B.Cu") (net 23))
 (segment (start 171 92.5) (end 172 91.5) (width 0.2) (layer "F.Cu") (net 35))
 (segment (start 165.5 91.05) (end 166.95 92.5) (width 0.2) (layer "F.Cu") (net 35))
 (segment (start 166.95 92.5) (end 171 92.5) (width 0.2) (layer "F.Cu") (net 35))
 (segment (start 172 91.5) (end 172 90.65) (width 0.2) (layer "F.Cu") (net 35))
 (segment (start 174 87) (end 172 89) (width 0.2) (layer "F.Cu") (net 20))
 (segment (start 170 89) (end 172 89) (width 0.2) (layer "F.Cu") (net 20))
 (segment (start 177.7 72.1) (end 174.9 72.1) (width 0.2) (layer "F.Cu") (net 20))
 (segment (start 174.9 72.1) (end 174 73) (width 0.2) (layer "F.Cu") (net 20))
 (segment (start 174 73) (end 174 87) (width 0.2) (layer "F.Cu") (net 20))
 (segment (start 160.52826 74.35) (end 159.00126 72.823) (width 0.2) (layer "F.Cu") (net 32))
 (segment (start 162.55 74.35) (end 160.52826 74.35) (width 0.2) (layer "F.Cu") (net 32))
 (segment (start 159.00126 72.823) (end 154.677 72.823) (width 0.2) (layer "F.Cu") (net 32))
 (segment (start 154.677 72.823) (end 153 74.5) (width 0.2) (layer "F.Cu") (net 32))
 (segment (start 162.55 76.89) (end 160.39 76.89) (width 0.2) (layer "F.Cu") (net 34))
 (segment (start 160.39 76.89) (end 158 74.5) (width 0.2) (layer "F.Cu") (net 34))
 (segment (start 162.55 75.62) (end 161.23116 75.62) (width 0.2) (layer "F.Cu") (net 33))
 (segment (start 161.23116 75.62) (end 158.83516 73.224) (width 0.2) (layer "F.Cu") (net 33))
 (segment (start 156.776 73.224) (end 155.5 74.5) (width 0.2) (layer "F.Cu") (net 33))
 (segment (start 158.83516 73.224) (end 156.776 73.224) (width 0.2) (layer "F.Cu") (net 33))
 (segment (start 152.578 72.422) (end 150.5 74.5) (width 0.2) (layer "F.Cu") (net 31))
 (segment (start 161.892 72.422) (end 152.578 72.422) (width 0.2) (layer "F.Cu") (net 31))
 (segment (start 162.55 73.08) (end 161.892 72.422) (width 0.2) (layer "F.Cu") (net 31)))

